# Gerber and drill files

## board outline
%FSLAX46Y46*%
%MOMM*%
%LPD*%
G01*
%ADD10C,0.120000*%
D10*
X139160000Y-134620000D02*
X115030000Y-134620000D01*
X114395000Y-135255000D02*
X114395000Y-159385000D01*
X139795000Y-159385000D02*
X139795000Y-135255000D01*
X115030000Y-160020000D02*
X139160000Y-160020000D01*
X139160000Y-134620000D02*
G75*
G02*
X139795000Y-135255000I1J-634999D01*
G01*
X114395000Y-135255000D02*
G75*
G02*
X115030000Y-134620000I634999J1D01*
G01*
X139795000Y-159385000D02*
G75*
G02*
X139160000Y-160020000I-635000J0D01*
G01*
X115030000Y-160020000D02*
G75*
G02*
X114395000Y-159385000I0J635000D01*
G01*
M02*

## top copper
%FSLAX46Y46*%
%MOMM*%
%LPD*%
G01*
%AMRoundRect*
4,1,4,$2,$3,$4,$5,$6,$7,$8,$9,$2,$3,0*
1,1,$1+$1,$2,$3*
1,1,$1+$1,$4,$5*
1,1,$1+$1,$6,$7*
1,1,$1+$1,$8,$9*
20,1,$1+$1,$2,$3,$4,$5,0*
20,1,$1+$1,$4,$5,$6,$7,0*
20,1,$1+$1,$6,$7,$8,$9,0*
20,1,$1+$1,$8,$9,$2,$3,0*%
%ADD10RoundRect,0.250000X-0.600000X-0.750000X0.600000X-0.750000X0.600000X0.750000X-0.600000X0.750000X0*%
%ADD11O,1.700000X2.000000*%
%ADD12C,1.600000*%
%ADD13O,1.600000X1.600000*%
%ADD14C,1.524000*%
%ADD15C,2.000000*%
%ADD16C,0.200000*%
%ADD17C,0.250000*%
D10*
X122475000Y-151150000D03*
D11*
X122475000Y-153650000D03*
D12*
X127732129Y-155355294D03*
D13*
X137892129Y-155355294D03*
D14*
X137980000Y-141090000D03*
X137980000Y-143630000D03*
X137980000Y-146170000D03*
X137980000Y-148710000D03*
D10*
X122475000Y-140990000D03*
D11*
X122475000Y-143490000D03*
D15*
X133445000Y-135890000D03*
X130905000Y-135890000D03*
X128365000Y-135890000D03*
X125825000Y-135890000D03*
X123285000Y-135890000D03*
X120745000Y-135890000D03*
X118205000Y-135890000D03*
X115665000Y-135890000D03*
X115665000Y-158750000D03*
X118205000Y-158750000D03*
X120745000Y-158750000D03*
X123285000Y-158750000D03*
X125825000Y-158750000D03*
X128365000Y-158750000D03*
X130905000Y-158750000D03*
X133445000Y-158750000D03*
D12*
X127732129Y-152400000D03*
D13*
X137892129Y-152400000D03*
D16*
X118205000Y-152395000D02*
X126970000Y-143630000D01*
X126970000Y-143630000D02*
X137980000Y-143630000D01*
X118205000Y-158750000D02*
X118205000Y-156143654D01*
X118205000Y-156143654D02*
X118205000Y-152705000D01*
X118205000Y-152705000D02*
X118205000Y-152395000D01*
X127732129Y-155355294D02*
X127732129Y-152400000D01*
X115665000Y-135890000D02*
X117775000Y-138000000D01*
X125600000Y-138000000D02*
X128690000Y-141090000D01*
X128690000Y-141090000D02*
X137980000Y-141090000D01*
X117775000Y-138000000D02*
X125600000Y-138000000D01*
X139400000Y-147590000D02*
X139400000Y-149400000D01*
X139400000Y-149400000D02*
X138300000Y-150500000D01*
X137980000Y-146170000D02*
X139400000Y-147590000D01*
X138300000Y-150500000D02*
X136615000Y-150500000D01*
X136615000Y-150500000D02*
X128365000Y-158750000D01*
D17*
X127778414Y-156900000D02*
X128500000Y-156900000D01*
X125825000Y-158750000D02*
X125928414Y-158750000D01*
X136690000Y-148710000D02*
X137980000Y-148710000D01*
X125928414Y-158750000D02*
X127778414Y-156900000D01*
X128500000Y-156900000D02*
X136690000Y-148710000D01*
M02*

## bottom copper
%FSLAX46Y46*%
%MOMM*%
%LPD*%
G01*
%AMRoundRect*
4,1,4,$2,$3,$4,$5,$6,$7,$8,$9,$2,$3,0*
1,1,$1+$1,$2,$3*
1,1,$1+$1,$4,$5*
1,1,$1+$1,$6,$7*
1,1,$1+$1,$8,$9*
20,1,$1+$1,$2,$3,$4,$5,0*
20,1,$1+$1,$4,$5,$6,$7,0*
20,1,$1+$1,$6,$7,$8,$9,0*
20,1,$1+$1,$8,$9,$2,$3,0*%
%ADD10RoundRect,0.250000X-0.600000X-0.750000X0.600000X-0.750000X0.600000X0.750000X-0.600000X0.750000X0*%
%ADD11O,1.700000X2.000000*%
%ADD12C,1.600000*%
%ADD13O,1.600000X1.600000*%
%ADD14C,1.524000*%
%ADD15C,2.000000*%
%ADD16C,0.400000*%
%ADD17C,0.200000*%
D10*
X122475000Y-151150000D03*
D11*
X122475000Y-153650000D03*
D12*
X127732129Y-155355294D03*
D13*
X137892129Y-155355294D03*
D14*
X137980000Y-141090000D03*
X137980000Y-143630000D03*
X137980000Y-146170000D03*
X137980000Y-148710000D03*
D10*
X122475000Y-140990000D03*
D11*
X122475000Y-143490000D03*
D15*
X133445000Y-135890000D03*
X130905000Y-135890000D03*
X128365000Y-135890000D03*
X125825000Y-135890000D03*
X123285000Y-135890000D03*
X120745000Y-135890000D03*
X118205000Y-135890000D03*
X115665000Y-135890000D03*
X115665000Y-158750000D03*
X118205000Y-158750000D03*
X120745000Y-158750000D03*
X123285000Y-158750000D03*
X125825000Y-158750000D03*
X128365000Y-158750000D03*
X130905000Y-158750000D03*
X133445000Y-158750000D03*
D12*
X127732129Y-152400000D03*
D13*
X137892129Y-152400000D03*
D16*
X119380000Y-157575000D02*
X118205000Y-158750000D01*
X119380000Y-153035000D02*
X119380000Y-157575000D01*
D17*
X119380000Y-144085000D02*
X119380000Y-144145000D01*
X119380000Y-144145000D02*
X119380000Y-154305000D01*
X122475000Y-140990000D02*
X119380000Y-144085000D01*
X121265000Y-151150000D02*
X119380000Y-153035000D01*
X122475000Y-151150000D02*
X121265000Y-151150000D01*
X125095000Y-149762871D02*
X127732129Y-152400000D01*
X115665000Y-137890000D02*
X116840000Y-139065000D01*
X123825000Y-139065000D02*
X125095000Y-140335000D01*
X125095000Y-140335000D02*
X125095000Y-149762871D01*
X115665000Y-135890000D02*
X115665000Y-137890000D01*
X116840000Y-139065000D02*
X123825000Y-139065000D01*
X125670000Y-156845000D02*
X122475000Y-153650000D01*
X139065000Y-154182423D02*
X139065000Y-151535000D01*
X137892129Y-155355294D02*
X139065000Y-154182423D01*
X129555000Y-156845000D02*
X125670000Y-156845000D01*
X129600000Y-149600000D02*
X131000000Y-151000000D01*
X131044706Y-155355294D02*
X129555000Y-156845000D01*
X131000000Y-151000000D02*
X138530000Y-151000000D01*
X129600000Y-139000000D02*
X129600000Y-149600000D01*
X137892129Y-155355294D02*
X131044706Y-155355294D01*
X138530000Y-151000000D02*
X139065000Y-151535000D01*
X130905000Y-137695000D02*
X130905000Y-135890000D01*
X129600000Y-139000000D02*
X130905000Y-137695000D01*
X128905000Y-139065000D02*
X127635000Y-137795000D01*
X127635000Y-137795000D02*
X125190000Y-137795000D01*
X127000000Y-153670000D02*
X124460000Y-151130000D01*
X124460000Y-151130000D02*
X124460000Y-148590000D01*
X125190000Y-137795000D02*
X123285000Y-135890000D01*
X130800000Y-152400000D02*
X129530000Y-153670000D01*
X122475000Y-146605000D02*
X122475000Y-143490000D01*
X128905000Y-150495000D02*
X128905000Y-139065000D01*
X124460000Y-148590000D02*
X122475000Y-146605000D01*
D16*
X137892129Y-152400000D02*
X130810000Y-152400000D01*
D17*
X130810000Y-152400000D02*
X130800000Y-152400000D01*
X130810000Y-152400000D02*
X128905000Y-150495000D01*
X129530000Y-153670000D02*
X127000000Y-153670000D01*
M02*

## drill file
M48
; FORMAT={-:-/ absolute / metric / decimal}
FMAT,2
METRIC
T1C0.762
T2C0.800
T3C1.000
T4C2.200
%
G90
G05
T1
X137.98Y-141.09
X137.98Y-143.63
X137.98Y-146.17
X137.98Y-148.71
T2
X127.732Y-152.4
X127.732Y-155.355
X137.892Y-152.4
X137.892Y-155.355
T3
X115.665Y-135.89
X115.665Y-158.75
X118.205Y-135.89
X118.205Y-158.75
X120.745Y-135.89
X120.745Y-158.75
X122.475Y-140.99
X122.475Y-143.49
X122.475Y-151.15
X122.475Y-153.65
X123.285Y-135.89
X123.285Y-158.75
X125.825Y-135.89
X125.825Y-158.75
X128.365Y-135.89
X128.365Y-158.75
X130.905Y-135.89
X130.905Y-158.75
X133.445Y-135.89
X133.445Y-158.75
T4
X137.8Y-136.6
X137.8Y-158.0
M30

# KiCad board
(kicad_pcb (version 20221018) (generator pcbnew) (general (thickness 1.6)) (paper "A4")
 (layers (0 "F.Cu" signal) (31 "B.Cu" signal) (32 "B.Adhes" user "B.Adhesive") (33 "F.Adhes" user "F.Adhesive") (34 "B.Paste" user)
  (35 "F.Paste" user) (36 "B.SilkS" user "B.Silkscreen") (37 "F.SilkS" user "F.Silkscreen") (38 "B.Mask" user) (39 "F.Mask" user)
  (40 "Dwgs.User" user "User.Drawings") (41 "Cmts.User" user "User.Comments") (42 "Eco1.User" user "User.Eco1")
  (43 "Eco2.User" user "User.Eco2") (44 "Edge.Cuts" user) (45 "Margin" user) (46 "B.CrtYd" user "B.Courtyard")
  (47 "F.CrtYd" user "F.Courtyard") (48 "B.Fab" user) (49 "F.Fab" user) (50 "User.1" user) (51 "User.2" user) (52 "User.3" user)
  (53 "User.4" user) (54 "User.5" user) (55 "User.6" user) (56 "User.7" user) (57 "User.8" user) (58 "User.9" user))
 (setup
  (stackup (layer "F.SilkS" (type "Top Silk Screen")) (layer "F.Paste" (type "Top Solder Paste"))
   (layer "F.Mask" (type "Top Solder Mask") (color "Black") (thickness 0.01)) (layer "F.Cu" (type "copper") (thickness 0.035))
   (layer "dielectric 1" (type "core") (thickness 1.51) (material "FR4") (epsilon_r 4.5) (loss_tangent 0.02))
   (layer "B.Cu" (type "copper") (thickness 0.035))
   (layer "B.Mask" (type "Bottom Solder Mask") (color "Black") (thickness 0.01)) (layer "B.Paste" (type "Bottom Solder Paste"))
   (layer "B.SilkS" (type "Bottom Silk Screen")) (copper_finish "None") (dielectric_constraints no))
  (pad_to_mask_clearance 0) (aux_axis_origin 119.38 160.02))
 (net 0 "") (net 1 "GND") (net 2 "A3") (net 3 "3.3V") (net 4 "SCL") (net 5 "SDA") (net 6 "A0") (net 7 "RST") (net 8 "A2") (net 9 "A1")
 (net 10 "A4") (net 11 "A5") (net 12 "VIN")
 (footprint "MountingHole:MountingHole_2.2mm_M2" (layer "F.Cu") (at 137.8 136.6)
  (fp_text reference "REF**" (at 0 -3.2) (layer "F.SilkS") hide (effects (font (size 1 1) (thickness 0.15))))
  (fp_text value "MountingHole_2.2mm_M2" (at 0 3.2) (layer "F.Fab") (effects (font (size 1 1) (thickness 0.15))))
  (pad "" np_thru_hole circle (at 0 0) (size 2.2 2.2) (drill 2.2) (layers "*.Cu" "*.Mask")))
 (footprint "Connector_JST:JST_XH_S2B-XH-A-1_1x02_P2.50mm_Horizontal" (layer "F.Cu") (at 114.375 152.4 -90)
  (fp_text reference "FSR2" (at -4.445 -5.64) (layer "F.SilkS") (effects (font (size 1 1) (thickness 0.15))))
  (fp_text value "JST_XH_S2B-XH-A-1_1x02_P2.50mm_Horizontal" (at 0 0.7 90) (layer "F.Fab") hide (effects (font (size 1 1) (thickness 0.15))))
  (pad "1" thru_hole roundrect (at -1.25 -8.1) (size 1.7 2) (drill 1) (layers "*.Cu" "*.Mask") (roundrect_rratio 0.1470588235) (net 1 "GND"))
  (pad "2" thru_hole oval (at 1.25 -8.1) (size 1.7 2) (drill 1) (layers "*.Cu" "*.Mask") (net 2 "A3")))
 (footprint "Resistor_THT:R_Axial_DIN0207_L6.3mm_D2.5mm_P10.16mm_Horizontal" (layer "F.Cu") (at 127.732129 155.355294)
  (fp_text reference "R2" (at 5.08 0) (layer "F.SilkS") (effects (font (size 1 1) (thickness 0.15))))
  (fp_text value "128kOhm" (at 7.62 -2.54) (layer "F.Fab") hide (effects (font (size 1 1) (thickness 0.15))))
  (pad "1" thru_hole circle (at 0 0) (size 1.6 1.6) (drill 0.8) (layers "*.Cu" "*.Mask") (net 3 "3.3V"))
  (pad "2" thru_hole oval (at 10.16 0) (size 1.6 1.6) (drill 0.8) (layers "*.Cu" "*.Mask") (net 2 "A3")))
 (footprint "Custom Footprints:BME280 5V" (layer "F.Cu") (at 136.71 144.9 -90)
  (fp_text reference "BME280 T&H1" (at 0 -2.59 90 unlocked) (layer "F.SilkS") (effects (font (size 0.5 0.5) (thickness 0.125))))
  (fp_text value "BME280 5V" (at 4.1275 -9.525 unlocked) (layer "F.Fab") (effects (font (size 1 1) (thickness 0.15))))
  (pad "1" thru_hole circle (at -3.81 -1.27 180) (size 1.524 1.524) (drill 0.762) (layers "*.Cu" "*.Mask") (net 3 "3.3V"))
  (pad "2" thru_hole circle (at -1.27 -1.27 180) (size 1.524 1.524) (drill 0.762) (layers "*.Cu" "*.Mask") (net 1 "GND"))
  (pad "3" thru_hole circle (at 1.27 -1.27 180) (size 1.524 1.524) (drill 0.762) (layers "*.Cu" "*.Mask") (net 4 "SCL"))
  (pad "4" thru_hole circle (at 3.81 -1.27 180) (size 1.524 1.524) (drill 0.762) (layers "*.Cu" "*.Mask") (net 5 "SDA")))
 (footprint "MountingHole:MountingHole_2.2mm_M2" (layer "F.Cu") (at 137.8 158)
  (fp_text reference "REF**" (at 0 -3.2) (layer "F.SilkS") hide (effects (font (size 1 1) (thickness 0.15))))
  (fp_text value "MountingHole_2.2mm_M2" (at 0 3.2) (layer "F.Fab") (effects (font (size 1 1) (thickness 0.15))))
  (pad "" np_thru_hole circle (at 0 0) (size 2.2 2.2) (drill 2.2) (layers "*.Cu" "*.Mask")))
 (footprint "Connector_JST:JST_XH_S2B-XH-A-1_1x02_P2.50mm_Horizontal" (layer "F.Cu") (at 114.375 142.24 -90)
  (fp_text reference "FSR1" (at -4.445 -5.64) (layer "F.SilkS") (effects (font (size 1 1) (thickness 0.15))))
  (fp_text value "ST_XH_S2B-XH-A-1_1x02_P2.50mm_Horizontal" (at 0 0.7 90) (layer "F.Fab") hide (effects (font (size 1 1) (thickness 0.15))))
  (pad "1" thru_hole roundrect (at -1.25 -8.1) (size 1.7 2) (drill 1) (layers "*.Cu" "*.Mask") (roundrect_rratio 0.1470588235) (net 1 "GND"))
  (pad "2" thru_hole oval (at 1.25 -8.1) (size 1.7 2) (drill 1) (layers "*.Cu" "*.Mask") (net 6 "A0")))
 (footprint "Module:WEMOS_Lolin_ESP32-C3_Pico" (layer "F.Cu") (at 114.395 147.32 -90)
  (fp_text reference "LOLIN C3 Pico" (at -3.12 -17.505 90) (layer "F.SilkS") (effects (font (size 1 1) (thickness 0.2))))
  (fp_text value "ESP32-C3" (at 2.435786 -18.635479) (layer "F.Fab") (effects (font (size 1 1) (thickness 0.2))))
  (fp_line (start -12.7 -24.765) (end -12.7 -0.635) (stroke (width 0.12) (type solid)) (layer "Edge.Cuts"))
  (fp_line (start -12.065 0) (end 12.065 0) (stroke (width 0.12) (type solid)) (layer "Edge.Cuts"))
  (fp_line (start 12.065 -25.4) (end -12.065 -25.4) (stroke (width 0.12) (type solid)) (layer "Edge.Cuts"))
  (fp_line (start 12.7 -0.635) (end 12.7 -24.765) (stroke (width 0.12) (type solid)) (layer "Edge.Cuts"))
  (fp_arc (start -12.7 -24.765) (mid -12.514013 -25.214013) (end -12.065 -25.4) (stroke (width 0.12) (type solid)) (layer "Edge.Cuts"))
  (fp_arc (start -12.065 0) (mid -12.514013 -0.185987) (end -12.7 -0.635) (stroke (width 0.12) (type solid)) (layer "Edge.Cuts"))
  (fp_arc (start 12.065 -25.4) (mid 12.514013 -25.214013) (end 12.7 -24.765) (stroke (width 0.12) (type solid)) (layer "Edge.Cuts"))
  (fp_arc (start 12.7 -0.635) (mid 12.514013 -0.185987) (end 12.065 0) (stroke (width 0.12) (type solid)) (layer "Edge.Cuts"))
  (pad "1" thru_hole circle (at -11.43 -19.05 270) (size 2 2) (drill 1) (layers "*.Cu" "*.Mask") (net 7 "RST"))
  (pad "2" thru_hole circle (at -11.43 -16.51 270) (size 2 2) (drill 1) (layers "*.Cu" "*.Mask") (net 2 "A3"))
  (pad "3" thru_hole circle (at -11.43 -13.97 270) (size 2 2) (drill 1) (layers "*.Cu" "*.Mask") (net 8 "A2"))
  (pad "4" thru_hole circle (at -11.43 -11.43 270) (size 2 2) (drill 1) (layers "*.Cu" "*.Mask") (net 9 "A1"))
  (pad "5" thru_hole circle (at -11.43 -8.89 270) (size 2 2) (drill 1) (layers "*.Cu" "*.Mask") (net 6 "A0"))
  (pad "6" thru_hole circle (at -11.43 -6.35 270) (size 2 2) (drill 1) (layers "*.Cu" "*.Mask") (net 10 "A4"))
  (pad "7" thru_hole circle (at -11.43 -3.81 270) (size 2 2) (drill 1) (layers "*.Cu" "*.Mask") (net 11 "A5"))
  (pad "8" thru_hole circle (at -11.43 -1.27 270) (size 2 2) (drill 1) (layers "*.Cu" "*.Mask") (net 3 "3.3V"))
  (pad "9" thru_hole circle (at 11.43 -1.27 270) (size 2 2) (drill 1) (layers "*.Cu" "*.Mask") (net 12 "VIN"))
  (pad "10" thru_hole circle (at 11.43 -3.81 270) (size 2 2) (drill 1) (layers "*.Cu" "*.Mask") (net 1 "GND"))
  (pad "11" thru_hole circle (at 11.43 -6.35 270) (size 2 2) (drill 1) (layers "*.Cu" "*.Mask"))
  (pad "12" thru_hole circle (at 11.43 -8.89 270) (size 2 2) (drill 1) (layers "*.Cu" "*.Mask"))
  (pad "13" thru_hole circle (at 11.43 -11.43 270) (size 2 2) (drill 1) (layers "*.Cu" "*.Mask") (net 5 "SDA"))
  (pad "14" thru_hole circle (at 11.43 -13.97 270) (size 2 2) (drill 1) (layers "*.Cu" "*.Mask") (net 4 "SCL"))
  (pad "15" thru_hole circle (at 11.43 -16.51 270) (size 2 2) (drill 1) (layers "*.Cu" "*.Mask"))
  (pad "16" thru_hole circle (at 11.43 -19.05 270) (size 2 2) (drill 1) (layers "*.Cu" "*.Mask")))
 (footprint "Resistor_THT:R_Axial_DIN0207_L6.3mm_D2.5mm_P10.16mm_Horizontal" (layer "F.Cu") (at 127.732129 152.4)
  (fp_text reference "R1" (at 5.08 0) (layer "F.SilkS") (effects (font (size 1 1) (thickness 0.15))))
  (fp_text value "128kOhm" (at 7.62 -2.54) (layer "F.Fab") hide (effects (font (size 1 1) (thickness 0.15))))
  (pad "1" thru_hole circle (at 0 0) (size 1.6 1.6) (drill 0.8) (layers "*.Cu" "*.Mask") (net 3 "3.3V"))
  (pad "2" thru_hole oval (at 10.16 0) (size 1.6 1.6) (drill 0.8) (layers "*.Cu" "*.Mask") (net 6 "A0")))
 (segment (start 118.205 152.395) (end 126.97 143.63) (width 0.2) (layer "F.Cu") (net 1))
 (segment (start 126.97 143.63) (end 137.98 143.63) (width 0.2) (layer "F.Cu") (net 1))
 (segment (start 118.205 158.75) (end 118.205 156.143654) (width 0.2) (layer "F.Cu") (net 1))
 (segment (start 118.205 156.143654) (end 118.205 152.705) (width 0.2) (layer "F.Cu") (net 1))
 (segment (start 118.205 152.705) (end 118.205 152.395) (width 0.2) (layer "F.Cu") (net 1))
 (segment (start 119.38 157.575) (end 118.205 158.75) (width 0.4) (layer "B.Cu") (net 1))
 (segment (start 119.38 153.035) (end 119.38 157.575) (width 0.4) (layer "B.Cu") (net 1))
 (segment (start 119.38 144.085) (end 119.38 144.145) (width 0.2) (layer "B.Cu") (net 1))
 (segment (start 119.38 144.145) (end 119.38 154.305) (width 0.2) (layer "B.Cu") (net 1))
 (segment (start 122.475 140.99) (end 119.38 144.085) (width 0.2) (layer "B.Cu") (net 1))
 (segment (start 121.265 151.15) (end 119.38 153.035) (width 0.2) (layer "B.Cu") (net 1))
 (segment (start 122.475 151.15) (end 121.265 151.15) (width 0.2) (layer "B.Cu") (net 1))
 (segment (start 127.732129 155.355294) (end 127.732129 152.4) (width 0.2) (layer "F.Cu") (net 3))
 (segment (start 115.665 135.89) (end 117.775 138) (width 0.2) (layer "F.Cu") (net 3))
 (segment (start 125.6 138) (end 128.69 141.09) (width 0.2) (layer "F.Cu") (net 3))
 (segment (start 128.69 141.09) (end 137.98 141.09) (width 0.2) (layer "F.Cu") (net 3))
 (segment (start 117.775 138) (end 125.6 138) (width 0.2) (layer "F.Cu") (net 3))
 (segment (start 125.095 149.762871) (end 127.732129 152.4) (width 0.2) (layer "B.Cu") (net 3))
 (segment (start 115.665 137.89) (end 116.84 139.065) (width 0.2) (layer "B.Cu") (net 3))
 (segment (start 123.825 139.065) (end 125.095 140.335) (width 0.2) (layer "B.Cu") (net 3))
 (segment (start 125.095 140.335) (end 125.095 149.762871) (width 0.2) (layer "B.Cu") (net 3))
 (segment (start 115.665 135.89) (end 115.665 137.89) (width 0.2) (layer "B.Cu") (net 3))
 (segment (start 116.84 139.065) (end 123.825 139.065) (width 0.2) (layer "B.Cu") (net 3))
 (segment (start 125.67 156.845) (end 122.475 153.65) (width 0.2) (layer "B.Cu") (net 2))
 (segment (start 139.065 154.182423) (end 139.065 151.535) (width 0.2) (layer "B.Cu") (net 2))
 (segment (start 137.892129 155.355294) (end 139.065 154.182423) (width 0.2) (layer "B.Cu") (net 2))
 (segment (start 129.555 156.845) (end 125.67 156.845) (width 0.2) (layer "B.Cu") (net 2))
 (segment (start 129.6 149.6) (end 131 151) (width 0.2) (layer "B.Cu") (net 2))
 (segment (start 131.044706 155.355294) (end 129.555 156.845) (width 0.2) (layer "B.Cu") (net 2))
 (segment (start 131 151) (end 138.53 151) (width 0.2) (layer "B.Cu") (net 2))
 (segment (start 129.6 139) (end 129.6 149.6) (width 0.2) (layer "B.Cu") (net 2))
 (segment (start 137.892129 155.355294) (end 131.044706 155.355294) (width 0.2) (layer "B.Cu") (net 2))
 (segment (start 138.53 151) (end 139.065 151.535) (width 0.2) (layer "B.Cu") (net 2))
 (segment (start 130.905 137.695) (end 130.905 135.89) (width 0.2) (layer "B.Cu") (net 2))
 (segment (start 129.6 139) (end 130.905 137.695) (width 0.2) (layer "B.Cu") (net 2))
 (segment (start 128.905 139.065) (end 127.635 137.795) (width 0.2) (layer "B.Cu") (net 6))
 (segment (start 127.635 137.795) (end 125.19 137.795) (width 0.2) (layer "B.Cu") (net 6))
 (segment (start 127 153.67) (end 124.46 151.13) (width 0.2) (layer "B.Cu") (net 6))
 (segment (start 124.46 151.13) (end 124.46 148.59) (width 0.2) (layer "B.Cu") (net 6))
 (segment (start 125.19 137.795) (end 123.285 135.89) (width 0.2) (layer "B.Cu") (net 6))
 (segment (start 130.8 152.4) (end 129.53 153.67) (width 0.2) (layer "B.Cu") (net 6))
 (segment (start 122.475 146.605) (end 122.475 143.49) (width 0.2) (layer "B.Cu") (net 6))
 (segment (start 128.905 150.495) (end 128.905 139.065) (width 0.2) (layer "B.Cu") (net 6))
 (segment (start 124.46 148.59) (end 122.475 146.605) (width 0.2) (layer "B.Cu") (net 6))
 (segment (start 137.892129 152.4) (end 130.81 152.4) (width 0.4) (layer "B.Cu") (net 6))
 (segment (start 130.81 152.4) (end 130.8 152.4) (width 0.2) (layer "B.Cu") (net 6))
 (segment (start 130.81 152.4) (end 128.905 150.495) (width 0.2) (layer "B.Cu") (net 6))
 (segment (start 129.53 153.67) (end 127 153.67) (width 0.2) (layer "B.Cu") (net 6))
 (segment (start 139.4 147.59) (end 139.4 149.4) (width 0.2) (layer "F.Cu") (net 4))
 (segment (start 139.4 149.4) (end 138.3 150.5) (width 0.2) (layer "F.Cu") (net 4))
 (segment (start 137.98 146.17) (end 139.4 147.59) (width 0.2) (layer "F.Cu") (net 4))
 (segment (start 138.3 150.5) (end 136.615 150.5) (width 0.2) (layer "F.Cu") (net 4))
 (segment (start 136.615 150.5) (end 128.365 158.75) (width 0.2) (layer "F.Cu") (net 4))
 (segment (start 127.778414 156.9) (end 128.5 156.9) (width 0.25) (layer "F.Cu") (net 5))
 (segment (start 125.825 158.75) (end 125.928414 158.75) (width 0.25) (layer "F.Cu") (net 5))
 (segment (start 136.69 148.71) (end 137.98 148.71) (width 0.25) (layer "F.Cu") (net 5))
 (segment (start 125.928414 158.75) (end 127.778414 156.9) (width 0.25) (layer "F.Cu") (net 5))
 (segment (start 128.5 156.9) (end 136.69 148.71) (width 0.25) (layer "F.Cu") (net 5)))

